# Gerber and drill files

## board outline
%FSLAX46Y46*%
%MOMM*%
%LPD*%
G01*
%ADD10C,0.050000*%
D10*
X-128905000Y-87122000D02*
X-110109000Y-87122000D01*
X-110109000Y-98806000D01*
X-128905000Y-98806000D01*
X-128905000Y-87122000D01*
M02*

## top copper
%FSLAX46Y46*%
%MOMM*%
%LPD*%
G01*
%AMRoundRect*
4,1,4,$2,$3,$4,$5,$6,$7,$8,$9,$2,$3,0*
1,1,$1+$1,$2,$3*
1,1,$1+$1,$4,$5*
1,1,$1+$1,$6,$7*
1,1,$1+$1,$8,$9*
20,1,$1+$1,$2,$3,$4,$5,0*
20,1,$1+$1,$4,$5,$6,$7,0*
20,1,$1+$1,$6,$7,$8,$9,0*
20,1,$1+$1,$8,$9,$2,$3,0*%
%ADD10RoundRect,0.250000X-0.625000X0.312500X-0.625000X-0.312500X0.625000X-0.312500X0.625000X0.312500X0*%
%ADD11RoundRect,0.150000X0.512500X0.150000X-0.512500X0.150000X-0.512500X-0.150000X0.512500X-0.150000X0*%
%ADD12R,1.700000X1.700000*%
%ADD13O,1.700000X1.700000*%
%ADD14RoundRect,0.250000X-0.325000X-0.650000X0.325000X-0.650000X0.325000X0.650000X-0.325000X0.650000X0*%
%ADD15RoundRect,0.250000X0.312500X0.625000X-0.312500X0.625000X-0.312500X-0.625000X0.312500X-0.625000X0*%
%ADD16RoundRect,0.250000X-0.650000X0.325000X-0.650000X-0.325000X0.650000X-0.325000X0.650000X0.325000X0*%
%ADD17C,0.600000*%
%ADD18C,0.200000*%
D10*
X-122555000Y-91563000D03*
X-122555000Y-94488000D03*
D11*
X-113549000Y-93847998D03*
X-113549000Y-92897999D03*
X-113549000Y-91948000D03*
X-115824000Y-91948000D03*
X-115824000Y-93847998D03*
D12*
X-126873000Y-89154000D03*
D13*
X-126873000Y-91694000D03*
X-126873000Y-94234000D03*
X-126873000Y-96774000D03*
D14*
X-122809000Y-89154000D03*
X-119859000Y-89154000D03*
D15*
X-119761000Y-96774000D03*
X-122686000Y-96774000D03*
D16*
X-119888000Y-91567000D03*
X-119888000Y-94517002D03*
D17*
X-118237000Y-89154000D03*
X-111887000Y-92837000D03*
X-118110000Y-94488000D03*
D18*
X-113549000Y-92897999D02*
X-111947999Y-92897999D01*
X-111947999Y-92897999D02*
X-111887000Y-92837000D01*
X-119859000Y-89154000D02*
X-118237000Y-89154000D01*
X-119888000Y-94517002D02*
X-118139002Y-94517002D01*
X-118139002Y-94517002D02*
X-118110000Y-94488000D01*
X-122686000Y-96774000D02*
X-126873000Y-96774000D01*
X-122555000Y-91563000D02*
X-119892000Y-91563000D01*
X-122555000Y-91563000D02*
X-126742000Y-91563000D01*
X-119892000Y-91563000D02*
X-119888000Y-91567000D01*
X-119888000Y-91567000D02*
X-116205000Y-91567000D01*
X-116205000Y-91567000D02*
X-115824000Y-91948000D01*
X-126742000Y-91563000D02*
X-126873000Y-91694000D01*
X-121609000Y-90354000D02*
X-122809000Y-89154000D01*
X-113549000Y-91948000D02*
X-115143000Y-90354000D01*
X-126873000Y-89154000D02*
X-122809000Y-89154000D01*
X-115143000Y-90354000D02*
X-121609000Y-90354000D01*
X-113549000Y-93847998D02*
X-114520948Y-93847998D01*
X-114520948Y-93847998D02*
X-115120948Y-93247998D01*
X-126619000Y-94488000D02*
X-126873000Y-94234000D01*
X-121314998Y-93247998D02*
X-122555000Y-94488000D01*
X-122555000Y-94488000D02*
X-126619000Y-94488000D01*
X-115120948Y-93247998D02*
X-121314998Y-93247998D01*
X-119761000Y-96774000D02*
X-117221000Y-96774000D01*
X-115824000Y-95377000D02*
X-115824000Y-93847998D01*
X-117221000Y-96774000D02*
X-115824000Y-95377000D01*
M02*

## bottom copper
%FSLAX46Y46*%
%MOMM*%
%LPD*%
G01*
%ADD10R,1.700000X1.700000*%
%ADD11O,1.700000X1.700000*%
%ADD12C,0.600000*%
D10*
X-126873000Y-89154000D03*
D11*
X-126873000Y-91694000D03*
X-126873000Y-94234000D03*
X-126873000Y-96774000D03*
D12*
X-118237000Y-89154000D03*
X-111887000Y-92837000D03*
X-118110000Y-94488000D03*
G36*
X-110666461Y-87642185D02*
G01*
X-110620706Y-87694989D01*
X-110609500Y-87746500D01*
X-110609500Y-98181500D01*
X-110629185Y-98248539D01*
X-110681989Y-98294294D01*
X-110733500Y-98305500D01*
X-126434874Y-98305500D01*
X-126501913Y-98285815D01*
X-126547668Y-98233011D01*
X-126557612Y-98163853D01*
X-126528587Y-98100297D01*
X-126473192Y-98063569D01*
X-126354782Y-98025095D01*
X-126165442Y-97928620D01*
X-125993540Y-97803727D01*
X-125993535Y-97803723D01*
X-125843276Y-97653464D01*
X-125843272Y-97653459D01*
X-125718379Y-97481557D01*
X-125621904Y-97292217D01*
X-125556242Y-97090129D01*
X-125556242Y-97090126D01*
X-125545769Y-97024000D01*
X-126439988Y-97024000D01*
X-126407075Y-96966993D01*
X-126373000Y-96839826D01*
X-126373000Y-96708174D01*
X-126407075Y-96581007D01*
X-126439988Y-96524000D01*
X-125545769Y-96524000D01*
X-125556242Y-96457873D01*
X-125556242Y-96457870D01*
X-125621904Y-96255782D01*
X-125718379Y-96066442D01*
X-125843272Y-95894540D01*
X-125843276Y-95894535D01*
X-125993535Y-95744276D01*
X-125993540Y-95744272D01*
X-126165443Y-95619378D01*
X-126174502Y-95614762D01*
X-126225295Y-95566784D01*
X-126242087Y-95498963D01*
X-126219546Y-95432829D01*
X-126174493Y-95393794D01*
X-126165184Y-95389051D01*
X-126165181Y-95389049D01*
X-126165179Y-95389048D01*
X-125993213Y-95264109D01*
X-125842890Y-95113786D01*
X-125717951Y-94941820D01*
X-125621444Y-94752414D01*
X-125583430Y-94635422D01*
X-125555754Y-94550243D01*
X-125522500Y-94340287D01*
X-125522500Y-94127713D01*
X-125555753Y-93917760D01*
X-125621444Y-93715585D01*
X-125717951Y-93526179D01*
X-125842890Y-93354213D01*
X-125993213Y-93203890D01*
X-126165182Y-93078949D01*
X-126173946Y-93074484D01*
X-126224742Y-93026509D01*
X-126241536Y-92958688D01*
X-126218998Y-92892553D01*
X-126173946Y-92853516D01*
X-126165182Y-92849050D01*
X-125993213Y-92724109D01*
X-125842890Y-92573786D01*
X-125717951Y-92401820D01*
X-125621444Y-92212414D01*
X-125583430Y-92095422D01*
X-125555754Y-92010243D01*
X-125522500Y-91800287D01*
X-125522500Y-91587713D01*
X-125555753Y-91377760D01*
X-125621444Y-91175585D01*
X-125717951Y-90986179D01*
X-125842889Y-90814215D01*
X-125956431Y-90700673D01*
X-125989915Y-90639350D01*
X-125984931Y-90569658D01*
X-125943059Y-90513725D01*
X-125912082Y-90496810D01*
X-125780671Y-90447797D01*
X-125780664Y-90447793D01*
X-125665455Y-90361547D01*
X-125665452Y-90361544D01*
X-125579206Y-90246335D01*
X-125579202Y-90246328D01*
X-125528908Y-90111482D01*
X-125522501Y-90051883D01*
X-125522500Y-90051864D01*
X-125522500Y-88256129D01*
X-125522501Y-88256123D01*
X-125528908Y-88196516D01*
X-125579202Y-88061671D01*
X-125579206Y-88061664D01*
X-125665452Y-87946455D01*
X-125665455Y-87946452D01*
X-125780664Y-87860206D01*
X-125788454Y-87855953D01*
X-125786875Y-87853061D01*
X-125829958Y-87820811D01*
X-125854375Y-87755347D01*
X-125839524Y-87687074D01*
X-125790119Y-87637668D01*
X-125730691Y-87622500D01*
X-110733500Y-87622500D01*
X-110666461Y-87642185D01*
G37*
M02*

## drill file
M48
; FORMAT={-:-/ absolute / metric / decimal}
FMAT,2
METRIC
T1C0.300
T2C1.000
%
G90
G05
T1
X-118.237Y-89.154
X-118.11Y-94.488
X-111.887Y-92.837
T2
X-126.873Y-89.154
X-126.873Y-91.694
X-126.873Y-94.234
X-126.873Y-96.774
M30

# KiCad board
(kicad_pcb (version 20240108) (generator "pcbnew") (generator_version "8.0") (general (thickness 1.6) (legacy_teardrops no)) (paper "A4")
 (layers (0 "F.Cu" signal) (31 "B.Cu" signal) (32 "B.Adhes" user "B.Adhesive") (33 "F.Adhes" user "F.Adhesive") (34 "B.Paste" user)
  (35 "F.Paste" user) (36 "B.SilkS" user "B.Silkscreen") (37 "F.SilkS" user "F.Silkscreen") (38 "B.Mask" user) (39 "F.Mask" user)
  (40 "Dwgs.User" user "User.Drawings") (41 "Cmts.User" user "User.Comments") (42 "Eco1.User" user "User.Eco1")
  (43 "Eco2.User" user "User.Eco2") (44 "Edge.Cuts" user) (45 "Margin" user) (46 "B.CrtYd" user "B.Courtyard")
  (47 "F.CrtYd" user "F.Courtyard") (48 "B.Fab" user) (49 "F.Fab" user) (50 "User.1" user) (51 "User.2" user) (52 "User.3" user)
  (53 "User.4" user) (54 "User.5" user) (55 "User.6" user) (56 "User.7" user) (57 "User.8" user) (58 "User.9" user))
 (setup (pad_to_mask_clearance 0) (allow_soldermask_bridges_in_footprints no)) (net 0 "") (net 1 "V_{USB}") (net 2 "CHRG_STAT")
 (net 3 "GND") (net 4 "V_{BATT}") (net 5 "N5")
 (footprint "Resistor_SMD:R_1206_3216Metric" (layer "F.Cu") (at -122.555 93.0255 -90)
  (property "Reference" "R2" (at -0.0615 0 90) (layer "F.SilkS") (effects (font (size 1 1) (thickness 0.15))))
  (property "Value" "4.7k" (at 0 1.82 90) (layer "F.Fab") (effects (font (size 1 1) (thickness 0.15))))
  (pad "1" smd roundrect (at -1.4625 0 270) (size 1.125 1.75) (layers "F.Cu" "F.Paste" "F.Mask") (roundrect_rratio 0.222222)
   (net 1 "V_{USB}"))
  (pad "2" smd roundrect (at 1.4625 0 270) (size 1.125 1.75) (layers "F.Cu" "F.Paste" "F.Mask") (roundrect_rratio 0.222222)
   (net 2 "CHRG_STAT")))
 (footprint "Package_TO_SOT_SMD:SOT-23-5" (layer "F.Cu") (at -114.6865 92.897999 180)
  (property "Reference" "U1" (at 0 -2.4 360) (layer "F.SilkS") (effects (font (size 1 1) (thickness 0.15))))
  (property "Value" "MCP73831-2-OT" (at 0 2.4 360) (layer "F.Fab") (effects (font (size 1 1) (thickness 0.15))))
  (pad "1" smd roundrect (at -1.1375 -0.949999 180) (size 1.325 0.6) (layers "F.Cu" "F.Paste" "F.Mask") (roundrect_rratio 0.25)
   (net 2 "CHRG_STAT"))
  (pad "2" smd roundrect (at -1.1375 0 180) (size 1.325 0.6) (layers "F.Cu" "F.Paste" "F.Mask") (roundrect_rratio 0.25) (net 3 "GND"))
  (pad "3" smd roundrect (at -1.1375 0.949999 180) (size 1.325 0.6) (layers "F.Cu" "F.Paste" "F.Mask") (roundrect_rratio 0.25)
   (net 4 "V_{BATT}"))
  (pad "4" smd roundrect (at 1.1375 0.949999 180) (size 1.325 0.6) (layers "F.Cu" "F.Paste" "F.Mask") (roundrect_rratio 0.25)
   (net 1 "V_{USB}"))
  (pad "5" smd roundrect (at 1.1375 -0.949999 180) (size 1.325 0.6) (layers "F.Cu" "F.Paste" "F.Mask") (roundrect_rratio 0.25) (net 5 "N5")))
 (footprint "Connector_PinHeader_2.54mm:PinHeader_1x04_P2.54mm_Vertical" (layer "F.Cu") (at -126.873 89.154)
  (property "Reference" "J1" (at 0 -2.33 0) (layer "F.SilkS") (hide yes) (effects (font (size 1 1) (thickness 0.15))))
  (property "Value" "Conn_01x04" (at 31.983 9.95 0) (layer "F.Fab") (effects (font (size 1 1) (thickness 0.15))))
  (pad "1" thru_hole rect (at 0 0) (size 1.7 1.7) (drill 1) (layers "*.Cu" "*.Mask") (remove_unused_layers no) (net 4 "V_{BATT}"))
  (pad "2" thru_hole oval (at 0 2.54) (size 1.7 1.7) (drill 1) (layers "*.Cu" "*.Mask") (remove_unused_layers no) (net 1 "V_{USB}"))
  (pad "3" thru_hole oval (at 0 5.08) (size 1.7 1.7) (drill 1) (layers "*.Cu" "*.Mask") (remove_unused_layers no) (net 2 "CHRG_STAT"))
  (pad "4" thru_hole oval (at 0 7.62) (size 1.7 1.7) (drill 1) (layers "*.Cu" "*.Mask") (remove_unused_layers no) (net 3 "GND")))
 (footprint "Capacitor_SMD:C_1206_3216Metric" (layer "F.Cu") (at -121.334 89.154)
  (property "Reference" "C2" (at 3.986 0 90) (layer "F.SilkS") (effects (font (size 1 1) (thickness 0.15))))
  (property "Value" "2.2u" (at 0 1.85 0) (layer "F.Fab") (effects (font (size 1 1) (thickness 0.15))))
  (pad "1" smd roundrect (at -1.475 0) (size 1.15 1.8) (layers "F.Cu" "F.Paste" "F.Mask") (roundrect_rratio 0.217391) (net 4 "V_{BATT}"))
  (pad "2" smd roundrect (at 1.475 0) (size 1.15 1.8) (layers "F.Cu" "F.Paste" "F.Mask") (roundrect_rratio 0.217391) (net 3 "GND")))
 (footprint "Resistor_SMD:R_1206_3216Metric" (layer "F.Cu") (at -121.2235 96.774 180)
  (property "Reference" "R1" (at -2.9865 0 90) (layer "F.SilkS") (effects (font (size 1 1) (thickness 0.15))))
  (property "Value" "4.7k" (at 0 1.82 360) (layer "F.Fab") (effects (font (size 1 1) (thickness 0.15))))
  (pad "1" smd roundrect (at -1.4625 0 180) (size 1.125 1.75) (layers "F.Cu" "F.Paste" "F.Mask") (roundrect_rratio 0.222222) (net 5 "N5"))
  (pad "2" smd roundrect (at 1.4625 0 180) (size 1.125 1.75) (layers "F.Cu" "F.Paste" "F.Mask") (roundrect_rratio 0.222222) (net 3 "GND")))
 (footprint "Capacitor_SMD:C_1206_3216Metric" (layer "F.Cu") (at -119.888 93.042001 -90)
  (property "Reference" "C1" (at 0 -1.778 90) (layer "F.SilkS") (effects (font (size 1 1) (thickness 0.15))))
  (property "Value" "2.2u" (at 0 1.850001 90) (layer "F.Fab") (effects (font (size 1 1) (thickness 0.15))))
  (pad "1" smd roundrect (at -1.475001 0 270) (size 1.15 1.8) (layers "F.Cu" "F.Paste" "F.Mask") (roundrect_rratio 0.217391)
   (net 1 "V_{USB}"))
  (pad "2" smd roundrect (at 1.475001 0 270) (size 1.15 1.8) (layers "F.Cu" "F.Paste" "F.Mask") (roundrect_rratio 0.217391) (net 3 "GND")))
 (gr_rect (start -128.905 87.122) (end -110.109 98.806) (stroke (width 0.05) (type default)) (fill none) (layer "Edge.Cuts"))
 (segment (start -113.549 92.897999) (end -111.947999 92.897999) (width 0.2) (layer "F.Cu") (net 3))
 (segment (start -111.947999 92.897999) (end -111.887 92.837) (width 0.2) (layer "F.Cu") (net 3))
 (segment (start -119.859 89.154) (end -118.237 89.154) (width 0.2) (layer "F.Cu") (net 3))
 (segment (start -119.888 94.517002) (end -118.139002 94.517002) (width 0.2) (layer "F.Cu") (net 3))
 (segment (start -118.139002 94.517002) (end -118.11 94.488) (width 0.2) (layer "F.Cu") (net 3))
 (segment (start -122.686 96.774) (end -126.873 96.774) (width 0.2) (layer "F.Cu") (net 3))
 (via (at -118.237 89.154) (size 0.6) (drill 0.3) (layers "F.Cu" "B.Cu") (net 3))
 (via (at -111.887 92.837) (size 0.6) (drill 0.3) (layers "F.Cu" "B.Cu") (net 3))
 (via (at -118.11 94.488) (size 0.6) (drill 0.3) (layers "F.Cu" "B.Cu") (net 3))
 (segment (start -122.555 91.563) (end -119.892 91.563) (width 0.2) (layer "F.Cu") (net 1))
 (segment (start -122.555 91.563) (end -126.742 91.563) (width 0.2) (layer "F.Cu") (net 1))
 (segment (start -119.892 91.563) (end -119.888 91.567) (width 0.2) (layer "F.Cu") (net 1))
 (segment (start -119.888 91.567) (end -116.205 91.567) (width 0.2) (layer "F.Cu") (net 1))
 (segment (start -116.205 91.567) (end -115.824 91.948) (width 0.2) (layer "F.Cu") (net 1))
 (segment (start -126.742 91.563) (end -126.873 91.694) (width 0.2) (layer "F.Cu") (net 1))
 (segment (start -121.609 90.354) (end -122.809 89.154) (width 0.2) (layer "F.Cu") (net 4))
 (segment (start -113.549 91.948) (end -115.143 90.354) (width 0.2) (layer "F.Cu") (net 4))
 (segment (start -126.873 89.154) (end -122.809 89.154) (width 0.2) (layer "F.Cu") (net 4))
 (segment (start -115.143 90.354) (end -121.609 90.354) (width 0.2) (layer "F.Cu") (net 4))
 (segment (start -113.549 93.847998) (end -114.520948 93.847998) (width 0.2) (layer "F.Cu") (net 2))
 (segment (start -114.520948 93.847998) (end -115.120948 93.247998) (width 0.2) (layer "F.Cu") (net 2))
 (segment (start -126.619 94.488) (end -126.873 94.234) (width 0.2) (layer "F.Cu") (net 2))
 (segment (start -121.314998 93.247998) (end -122.555 94.488) (width 0.2) (layer "F.Cu") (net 2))
 (segment (start -122.555 94.488) (end -126.619 94.488) (width 0.2) (layer "F.Cu") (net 2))
 (segment (start -115.120948 93.247998) (end -121.314998 93.247998) (width 0.2) (layer "F.Cu") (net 2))
 (segment (start -119.761 96.774) (end -117.221 96.774) (width 0.2) (layer "F.Cu") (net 5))
 (segment (start -115.824 95.377) (end -115.824 93.847998) (width 0.2) (layer "F.Cu") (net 5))
 (segment (start -117.221 96.774) (end -115.824 95.377) (width 0.2) (layer "F.Cu") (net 5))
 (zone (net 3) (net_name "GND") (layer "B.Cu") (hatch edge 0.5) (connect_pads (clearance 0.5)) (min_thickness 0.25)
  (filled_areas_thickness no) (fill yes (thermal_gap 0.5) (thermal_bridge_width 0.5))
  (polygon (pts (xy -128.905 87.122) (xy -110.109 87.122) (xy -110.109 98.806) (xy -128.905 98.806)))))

